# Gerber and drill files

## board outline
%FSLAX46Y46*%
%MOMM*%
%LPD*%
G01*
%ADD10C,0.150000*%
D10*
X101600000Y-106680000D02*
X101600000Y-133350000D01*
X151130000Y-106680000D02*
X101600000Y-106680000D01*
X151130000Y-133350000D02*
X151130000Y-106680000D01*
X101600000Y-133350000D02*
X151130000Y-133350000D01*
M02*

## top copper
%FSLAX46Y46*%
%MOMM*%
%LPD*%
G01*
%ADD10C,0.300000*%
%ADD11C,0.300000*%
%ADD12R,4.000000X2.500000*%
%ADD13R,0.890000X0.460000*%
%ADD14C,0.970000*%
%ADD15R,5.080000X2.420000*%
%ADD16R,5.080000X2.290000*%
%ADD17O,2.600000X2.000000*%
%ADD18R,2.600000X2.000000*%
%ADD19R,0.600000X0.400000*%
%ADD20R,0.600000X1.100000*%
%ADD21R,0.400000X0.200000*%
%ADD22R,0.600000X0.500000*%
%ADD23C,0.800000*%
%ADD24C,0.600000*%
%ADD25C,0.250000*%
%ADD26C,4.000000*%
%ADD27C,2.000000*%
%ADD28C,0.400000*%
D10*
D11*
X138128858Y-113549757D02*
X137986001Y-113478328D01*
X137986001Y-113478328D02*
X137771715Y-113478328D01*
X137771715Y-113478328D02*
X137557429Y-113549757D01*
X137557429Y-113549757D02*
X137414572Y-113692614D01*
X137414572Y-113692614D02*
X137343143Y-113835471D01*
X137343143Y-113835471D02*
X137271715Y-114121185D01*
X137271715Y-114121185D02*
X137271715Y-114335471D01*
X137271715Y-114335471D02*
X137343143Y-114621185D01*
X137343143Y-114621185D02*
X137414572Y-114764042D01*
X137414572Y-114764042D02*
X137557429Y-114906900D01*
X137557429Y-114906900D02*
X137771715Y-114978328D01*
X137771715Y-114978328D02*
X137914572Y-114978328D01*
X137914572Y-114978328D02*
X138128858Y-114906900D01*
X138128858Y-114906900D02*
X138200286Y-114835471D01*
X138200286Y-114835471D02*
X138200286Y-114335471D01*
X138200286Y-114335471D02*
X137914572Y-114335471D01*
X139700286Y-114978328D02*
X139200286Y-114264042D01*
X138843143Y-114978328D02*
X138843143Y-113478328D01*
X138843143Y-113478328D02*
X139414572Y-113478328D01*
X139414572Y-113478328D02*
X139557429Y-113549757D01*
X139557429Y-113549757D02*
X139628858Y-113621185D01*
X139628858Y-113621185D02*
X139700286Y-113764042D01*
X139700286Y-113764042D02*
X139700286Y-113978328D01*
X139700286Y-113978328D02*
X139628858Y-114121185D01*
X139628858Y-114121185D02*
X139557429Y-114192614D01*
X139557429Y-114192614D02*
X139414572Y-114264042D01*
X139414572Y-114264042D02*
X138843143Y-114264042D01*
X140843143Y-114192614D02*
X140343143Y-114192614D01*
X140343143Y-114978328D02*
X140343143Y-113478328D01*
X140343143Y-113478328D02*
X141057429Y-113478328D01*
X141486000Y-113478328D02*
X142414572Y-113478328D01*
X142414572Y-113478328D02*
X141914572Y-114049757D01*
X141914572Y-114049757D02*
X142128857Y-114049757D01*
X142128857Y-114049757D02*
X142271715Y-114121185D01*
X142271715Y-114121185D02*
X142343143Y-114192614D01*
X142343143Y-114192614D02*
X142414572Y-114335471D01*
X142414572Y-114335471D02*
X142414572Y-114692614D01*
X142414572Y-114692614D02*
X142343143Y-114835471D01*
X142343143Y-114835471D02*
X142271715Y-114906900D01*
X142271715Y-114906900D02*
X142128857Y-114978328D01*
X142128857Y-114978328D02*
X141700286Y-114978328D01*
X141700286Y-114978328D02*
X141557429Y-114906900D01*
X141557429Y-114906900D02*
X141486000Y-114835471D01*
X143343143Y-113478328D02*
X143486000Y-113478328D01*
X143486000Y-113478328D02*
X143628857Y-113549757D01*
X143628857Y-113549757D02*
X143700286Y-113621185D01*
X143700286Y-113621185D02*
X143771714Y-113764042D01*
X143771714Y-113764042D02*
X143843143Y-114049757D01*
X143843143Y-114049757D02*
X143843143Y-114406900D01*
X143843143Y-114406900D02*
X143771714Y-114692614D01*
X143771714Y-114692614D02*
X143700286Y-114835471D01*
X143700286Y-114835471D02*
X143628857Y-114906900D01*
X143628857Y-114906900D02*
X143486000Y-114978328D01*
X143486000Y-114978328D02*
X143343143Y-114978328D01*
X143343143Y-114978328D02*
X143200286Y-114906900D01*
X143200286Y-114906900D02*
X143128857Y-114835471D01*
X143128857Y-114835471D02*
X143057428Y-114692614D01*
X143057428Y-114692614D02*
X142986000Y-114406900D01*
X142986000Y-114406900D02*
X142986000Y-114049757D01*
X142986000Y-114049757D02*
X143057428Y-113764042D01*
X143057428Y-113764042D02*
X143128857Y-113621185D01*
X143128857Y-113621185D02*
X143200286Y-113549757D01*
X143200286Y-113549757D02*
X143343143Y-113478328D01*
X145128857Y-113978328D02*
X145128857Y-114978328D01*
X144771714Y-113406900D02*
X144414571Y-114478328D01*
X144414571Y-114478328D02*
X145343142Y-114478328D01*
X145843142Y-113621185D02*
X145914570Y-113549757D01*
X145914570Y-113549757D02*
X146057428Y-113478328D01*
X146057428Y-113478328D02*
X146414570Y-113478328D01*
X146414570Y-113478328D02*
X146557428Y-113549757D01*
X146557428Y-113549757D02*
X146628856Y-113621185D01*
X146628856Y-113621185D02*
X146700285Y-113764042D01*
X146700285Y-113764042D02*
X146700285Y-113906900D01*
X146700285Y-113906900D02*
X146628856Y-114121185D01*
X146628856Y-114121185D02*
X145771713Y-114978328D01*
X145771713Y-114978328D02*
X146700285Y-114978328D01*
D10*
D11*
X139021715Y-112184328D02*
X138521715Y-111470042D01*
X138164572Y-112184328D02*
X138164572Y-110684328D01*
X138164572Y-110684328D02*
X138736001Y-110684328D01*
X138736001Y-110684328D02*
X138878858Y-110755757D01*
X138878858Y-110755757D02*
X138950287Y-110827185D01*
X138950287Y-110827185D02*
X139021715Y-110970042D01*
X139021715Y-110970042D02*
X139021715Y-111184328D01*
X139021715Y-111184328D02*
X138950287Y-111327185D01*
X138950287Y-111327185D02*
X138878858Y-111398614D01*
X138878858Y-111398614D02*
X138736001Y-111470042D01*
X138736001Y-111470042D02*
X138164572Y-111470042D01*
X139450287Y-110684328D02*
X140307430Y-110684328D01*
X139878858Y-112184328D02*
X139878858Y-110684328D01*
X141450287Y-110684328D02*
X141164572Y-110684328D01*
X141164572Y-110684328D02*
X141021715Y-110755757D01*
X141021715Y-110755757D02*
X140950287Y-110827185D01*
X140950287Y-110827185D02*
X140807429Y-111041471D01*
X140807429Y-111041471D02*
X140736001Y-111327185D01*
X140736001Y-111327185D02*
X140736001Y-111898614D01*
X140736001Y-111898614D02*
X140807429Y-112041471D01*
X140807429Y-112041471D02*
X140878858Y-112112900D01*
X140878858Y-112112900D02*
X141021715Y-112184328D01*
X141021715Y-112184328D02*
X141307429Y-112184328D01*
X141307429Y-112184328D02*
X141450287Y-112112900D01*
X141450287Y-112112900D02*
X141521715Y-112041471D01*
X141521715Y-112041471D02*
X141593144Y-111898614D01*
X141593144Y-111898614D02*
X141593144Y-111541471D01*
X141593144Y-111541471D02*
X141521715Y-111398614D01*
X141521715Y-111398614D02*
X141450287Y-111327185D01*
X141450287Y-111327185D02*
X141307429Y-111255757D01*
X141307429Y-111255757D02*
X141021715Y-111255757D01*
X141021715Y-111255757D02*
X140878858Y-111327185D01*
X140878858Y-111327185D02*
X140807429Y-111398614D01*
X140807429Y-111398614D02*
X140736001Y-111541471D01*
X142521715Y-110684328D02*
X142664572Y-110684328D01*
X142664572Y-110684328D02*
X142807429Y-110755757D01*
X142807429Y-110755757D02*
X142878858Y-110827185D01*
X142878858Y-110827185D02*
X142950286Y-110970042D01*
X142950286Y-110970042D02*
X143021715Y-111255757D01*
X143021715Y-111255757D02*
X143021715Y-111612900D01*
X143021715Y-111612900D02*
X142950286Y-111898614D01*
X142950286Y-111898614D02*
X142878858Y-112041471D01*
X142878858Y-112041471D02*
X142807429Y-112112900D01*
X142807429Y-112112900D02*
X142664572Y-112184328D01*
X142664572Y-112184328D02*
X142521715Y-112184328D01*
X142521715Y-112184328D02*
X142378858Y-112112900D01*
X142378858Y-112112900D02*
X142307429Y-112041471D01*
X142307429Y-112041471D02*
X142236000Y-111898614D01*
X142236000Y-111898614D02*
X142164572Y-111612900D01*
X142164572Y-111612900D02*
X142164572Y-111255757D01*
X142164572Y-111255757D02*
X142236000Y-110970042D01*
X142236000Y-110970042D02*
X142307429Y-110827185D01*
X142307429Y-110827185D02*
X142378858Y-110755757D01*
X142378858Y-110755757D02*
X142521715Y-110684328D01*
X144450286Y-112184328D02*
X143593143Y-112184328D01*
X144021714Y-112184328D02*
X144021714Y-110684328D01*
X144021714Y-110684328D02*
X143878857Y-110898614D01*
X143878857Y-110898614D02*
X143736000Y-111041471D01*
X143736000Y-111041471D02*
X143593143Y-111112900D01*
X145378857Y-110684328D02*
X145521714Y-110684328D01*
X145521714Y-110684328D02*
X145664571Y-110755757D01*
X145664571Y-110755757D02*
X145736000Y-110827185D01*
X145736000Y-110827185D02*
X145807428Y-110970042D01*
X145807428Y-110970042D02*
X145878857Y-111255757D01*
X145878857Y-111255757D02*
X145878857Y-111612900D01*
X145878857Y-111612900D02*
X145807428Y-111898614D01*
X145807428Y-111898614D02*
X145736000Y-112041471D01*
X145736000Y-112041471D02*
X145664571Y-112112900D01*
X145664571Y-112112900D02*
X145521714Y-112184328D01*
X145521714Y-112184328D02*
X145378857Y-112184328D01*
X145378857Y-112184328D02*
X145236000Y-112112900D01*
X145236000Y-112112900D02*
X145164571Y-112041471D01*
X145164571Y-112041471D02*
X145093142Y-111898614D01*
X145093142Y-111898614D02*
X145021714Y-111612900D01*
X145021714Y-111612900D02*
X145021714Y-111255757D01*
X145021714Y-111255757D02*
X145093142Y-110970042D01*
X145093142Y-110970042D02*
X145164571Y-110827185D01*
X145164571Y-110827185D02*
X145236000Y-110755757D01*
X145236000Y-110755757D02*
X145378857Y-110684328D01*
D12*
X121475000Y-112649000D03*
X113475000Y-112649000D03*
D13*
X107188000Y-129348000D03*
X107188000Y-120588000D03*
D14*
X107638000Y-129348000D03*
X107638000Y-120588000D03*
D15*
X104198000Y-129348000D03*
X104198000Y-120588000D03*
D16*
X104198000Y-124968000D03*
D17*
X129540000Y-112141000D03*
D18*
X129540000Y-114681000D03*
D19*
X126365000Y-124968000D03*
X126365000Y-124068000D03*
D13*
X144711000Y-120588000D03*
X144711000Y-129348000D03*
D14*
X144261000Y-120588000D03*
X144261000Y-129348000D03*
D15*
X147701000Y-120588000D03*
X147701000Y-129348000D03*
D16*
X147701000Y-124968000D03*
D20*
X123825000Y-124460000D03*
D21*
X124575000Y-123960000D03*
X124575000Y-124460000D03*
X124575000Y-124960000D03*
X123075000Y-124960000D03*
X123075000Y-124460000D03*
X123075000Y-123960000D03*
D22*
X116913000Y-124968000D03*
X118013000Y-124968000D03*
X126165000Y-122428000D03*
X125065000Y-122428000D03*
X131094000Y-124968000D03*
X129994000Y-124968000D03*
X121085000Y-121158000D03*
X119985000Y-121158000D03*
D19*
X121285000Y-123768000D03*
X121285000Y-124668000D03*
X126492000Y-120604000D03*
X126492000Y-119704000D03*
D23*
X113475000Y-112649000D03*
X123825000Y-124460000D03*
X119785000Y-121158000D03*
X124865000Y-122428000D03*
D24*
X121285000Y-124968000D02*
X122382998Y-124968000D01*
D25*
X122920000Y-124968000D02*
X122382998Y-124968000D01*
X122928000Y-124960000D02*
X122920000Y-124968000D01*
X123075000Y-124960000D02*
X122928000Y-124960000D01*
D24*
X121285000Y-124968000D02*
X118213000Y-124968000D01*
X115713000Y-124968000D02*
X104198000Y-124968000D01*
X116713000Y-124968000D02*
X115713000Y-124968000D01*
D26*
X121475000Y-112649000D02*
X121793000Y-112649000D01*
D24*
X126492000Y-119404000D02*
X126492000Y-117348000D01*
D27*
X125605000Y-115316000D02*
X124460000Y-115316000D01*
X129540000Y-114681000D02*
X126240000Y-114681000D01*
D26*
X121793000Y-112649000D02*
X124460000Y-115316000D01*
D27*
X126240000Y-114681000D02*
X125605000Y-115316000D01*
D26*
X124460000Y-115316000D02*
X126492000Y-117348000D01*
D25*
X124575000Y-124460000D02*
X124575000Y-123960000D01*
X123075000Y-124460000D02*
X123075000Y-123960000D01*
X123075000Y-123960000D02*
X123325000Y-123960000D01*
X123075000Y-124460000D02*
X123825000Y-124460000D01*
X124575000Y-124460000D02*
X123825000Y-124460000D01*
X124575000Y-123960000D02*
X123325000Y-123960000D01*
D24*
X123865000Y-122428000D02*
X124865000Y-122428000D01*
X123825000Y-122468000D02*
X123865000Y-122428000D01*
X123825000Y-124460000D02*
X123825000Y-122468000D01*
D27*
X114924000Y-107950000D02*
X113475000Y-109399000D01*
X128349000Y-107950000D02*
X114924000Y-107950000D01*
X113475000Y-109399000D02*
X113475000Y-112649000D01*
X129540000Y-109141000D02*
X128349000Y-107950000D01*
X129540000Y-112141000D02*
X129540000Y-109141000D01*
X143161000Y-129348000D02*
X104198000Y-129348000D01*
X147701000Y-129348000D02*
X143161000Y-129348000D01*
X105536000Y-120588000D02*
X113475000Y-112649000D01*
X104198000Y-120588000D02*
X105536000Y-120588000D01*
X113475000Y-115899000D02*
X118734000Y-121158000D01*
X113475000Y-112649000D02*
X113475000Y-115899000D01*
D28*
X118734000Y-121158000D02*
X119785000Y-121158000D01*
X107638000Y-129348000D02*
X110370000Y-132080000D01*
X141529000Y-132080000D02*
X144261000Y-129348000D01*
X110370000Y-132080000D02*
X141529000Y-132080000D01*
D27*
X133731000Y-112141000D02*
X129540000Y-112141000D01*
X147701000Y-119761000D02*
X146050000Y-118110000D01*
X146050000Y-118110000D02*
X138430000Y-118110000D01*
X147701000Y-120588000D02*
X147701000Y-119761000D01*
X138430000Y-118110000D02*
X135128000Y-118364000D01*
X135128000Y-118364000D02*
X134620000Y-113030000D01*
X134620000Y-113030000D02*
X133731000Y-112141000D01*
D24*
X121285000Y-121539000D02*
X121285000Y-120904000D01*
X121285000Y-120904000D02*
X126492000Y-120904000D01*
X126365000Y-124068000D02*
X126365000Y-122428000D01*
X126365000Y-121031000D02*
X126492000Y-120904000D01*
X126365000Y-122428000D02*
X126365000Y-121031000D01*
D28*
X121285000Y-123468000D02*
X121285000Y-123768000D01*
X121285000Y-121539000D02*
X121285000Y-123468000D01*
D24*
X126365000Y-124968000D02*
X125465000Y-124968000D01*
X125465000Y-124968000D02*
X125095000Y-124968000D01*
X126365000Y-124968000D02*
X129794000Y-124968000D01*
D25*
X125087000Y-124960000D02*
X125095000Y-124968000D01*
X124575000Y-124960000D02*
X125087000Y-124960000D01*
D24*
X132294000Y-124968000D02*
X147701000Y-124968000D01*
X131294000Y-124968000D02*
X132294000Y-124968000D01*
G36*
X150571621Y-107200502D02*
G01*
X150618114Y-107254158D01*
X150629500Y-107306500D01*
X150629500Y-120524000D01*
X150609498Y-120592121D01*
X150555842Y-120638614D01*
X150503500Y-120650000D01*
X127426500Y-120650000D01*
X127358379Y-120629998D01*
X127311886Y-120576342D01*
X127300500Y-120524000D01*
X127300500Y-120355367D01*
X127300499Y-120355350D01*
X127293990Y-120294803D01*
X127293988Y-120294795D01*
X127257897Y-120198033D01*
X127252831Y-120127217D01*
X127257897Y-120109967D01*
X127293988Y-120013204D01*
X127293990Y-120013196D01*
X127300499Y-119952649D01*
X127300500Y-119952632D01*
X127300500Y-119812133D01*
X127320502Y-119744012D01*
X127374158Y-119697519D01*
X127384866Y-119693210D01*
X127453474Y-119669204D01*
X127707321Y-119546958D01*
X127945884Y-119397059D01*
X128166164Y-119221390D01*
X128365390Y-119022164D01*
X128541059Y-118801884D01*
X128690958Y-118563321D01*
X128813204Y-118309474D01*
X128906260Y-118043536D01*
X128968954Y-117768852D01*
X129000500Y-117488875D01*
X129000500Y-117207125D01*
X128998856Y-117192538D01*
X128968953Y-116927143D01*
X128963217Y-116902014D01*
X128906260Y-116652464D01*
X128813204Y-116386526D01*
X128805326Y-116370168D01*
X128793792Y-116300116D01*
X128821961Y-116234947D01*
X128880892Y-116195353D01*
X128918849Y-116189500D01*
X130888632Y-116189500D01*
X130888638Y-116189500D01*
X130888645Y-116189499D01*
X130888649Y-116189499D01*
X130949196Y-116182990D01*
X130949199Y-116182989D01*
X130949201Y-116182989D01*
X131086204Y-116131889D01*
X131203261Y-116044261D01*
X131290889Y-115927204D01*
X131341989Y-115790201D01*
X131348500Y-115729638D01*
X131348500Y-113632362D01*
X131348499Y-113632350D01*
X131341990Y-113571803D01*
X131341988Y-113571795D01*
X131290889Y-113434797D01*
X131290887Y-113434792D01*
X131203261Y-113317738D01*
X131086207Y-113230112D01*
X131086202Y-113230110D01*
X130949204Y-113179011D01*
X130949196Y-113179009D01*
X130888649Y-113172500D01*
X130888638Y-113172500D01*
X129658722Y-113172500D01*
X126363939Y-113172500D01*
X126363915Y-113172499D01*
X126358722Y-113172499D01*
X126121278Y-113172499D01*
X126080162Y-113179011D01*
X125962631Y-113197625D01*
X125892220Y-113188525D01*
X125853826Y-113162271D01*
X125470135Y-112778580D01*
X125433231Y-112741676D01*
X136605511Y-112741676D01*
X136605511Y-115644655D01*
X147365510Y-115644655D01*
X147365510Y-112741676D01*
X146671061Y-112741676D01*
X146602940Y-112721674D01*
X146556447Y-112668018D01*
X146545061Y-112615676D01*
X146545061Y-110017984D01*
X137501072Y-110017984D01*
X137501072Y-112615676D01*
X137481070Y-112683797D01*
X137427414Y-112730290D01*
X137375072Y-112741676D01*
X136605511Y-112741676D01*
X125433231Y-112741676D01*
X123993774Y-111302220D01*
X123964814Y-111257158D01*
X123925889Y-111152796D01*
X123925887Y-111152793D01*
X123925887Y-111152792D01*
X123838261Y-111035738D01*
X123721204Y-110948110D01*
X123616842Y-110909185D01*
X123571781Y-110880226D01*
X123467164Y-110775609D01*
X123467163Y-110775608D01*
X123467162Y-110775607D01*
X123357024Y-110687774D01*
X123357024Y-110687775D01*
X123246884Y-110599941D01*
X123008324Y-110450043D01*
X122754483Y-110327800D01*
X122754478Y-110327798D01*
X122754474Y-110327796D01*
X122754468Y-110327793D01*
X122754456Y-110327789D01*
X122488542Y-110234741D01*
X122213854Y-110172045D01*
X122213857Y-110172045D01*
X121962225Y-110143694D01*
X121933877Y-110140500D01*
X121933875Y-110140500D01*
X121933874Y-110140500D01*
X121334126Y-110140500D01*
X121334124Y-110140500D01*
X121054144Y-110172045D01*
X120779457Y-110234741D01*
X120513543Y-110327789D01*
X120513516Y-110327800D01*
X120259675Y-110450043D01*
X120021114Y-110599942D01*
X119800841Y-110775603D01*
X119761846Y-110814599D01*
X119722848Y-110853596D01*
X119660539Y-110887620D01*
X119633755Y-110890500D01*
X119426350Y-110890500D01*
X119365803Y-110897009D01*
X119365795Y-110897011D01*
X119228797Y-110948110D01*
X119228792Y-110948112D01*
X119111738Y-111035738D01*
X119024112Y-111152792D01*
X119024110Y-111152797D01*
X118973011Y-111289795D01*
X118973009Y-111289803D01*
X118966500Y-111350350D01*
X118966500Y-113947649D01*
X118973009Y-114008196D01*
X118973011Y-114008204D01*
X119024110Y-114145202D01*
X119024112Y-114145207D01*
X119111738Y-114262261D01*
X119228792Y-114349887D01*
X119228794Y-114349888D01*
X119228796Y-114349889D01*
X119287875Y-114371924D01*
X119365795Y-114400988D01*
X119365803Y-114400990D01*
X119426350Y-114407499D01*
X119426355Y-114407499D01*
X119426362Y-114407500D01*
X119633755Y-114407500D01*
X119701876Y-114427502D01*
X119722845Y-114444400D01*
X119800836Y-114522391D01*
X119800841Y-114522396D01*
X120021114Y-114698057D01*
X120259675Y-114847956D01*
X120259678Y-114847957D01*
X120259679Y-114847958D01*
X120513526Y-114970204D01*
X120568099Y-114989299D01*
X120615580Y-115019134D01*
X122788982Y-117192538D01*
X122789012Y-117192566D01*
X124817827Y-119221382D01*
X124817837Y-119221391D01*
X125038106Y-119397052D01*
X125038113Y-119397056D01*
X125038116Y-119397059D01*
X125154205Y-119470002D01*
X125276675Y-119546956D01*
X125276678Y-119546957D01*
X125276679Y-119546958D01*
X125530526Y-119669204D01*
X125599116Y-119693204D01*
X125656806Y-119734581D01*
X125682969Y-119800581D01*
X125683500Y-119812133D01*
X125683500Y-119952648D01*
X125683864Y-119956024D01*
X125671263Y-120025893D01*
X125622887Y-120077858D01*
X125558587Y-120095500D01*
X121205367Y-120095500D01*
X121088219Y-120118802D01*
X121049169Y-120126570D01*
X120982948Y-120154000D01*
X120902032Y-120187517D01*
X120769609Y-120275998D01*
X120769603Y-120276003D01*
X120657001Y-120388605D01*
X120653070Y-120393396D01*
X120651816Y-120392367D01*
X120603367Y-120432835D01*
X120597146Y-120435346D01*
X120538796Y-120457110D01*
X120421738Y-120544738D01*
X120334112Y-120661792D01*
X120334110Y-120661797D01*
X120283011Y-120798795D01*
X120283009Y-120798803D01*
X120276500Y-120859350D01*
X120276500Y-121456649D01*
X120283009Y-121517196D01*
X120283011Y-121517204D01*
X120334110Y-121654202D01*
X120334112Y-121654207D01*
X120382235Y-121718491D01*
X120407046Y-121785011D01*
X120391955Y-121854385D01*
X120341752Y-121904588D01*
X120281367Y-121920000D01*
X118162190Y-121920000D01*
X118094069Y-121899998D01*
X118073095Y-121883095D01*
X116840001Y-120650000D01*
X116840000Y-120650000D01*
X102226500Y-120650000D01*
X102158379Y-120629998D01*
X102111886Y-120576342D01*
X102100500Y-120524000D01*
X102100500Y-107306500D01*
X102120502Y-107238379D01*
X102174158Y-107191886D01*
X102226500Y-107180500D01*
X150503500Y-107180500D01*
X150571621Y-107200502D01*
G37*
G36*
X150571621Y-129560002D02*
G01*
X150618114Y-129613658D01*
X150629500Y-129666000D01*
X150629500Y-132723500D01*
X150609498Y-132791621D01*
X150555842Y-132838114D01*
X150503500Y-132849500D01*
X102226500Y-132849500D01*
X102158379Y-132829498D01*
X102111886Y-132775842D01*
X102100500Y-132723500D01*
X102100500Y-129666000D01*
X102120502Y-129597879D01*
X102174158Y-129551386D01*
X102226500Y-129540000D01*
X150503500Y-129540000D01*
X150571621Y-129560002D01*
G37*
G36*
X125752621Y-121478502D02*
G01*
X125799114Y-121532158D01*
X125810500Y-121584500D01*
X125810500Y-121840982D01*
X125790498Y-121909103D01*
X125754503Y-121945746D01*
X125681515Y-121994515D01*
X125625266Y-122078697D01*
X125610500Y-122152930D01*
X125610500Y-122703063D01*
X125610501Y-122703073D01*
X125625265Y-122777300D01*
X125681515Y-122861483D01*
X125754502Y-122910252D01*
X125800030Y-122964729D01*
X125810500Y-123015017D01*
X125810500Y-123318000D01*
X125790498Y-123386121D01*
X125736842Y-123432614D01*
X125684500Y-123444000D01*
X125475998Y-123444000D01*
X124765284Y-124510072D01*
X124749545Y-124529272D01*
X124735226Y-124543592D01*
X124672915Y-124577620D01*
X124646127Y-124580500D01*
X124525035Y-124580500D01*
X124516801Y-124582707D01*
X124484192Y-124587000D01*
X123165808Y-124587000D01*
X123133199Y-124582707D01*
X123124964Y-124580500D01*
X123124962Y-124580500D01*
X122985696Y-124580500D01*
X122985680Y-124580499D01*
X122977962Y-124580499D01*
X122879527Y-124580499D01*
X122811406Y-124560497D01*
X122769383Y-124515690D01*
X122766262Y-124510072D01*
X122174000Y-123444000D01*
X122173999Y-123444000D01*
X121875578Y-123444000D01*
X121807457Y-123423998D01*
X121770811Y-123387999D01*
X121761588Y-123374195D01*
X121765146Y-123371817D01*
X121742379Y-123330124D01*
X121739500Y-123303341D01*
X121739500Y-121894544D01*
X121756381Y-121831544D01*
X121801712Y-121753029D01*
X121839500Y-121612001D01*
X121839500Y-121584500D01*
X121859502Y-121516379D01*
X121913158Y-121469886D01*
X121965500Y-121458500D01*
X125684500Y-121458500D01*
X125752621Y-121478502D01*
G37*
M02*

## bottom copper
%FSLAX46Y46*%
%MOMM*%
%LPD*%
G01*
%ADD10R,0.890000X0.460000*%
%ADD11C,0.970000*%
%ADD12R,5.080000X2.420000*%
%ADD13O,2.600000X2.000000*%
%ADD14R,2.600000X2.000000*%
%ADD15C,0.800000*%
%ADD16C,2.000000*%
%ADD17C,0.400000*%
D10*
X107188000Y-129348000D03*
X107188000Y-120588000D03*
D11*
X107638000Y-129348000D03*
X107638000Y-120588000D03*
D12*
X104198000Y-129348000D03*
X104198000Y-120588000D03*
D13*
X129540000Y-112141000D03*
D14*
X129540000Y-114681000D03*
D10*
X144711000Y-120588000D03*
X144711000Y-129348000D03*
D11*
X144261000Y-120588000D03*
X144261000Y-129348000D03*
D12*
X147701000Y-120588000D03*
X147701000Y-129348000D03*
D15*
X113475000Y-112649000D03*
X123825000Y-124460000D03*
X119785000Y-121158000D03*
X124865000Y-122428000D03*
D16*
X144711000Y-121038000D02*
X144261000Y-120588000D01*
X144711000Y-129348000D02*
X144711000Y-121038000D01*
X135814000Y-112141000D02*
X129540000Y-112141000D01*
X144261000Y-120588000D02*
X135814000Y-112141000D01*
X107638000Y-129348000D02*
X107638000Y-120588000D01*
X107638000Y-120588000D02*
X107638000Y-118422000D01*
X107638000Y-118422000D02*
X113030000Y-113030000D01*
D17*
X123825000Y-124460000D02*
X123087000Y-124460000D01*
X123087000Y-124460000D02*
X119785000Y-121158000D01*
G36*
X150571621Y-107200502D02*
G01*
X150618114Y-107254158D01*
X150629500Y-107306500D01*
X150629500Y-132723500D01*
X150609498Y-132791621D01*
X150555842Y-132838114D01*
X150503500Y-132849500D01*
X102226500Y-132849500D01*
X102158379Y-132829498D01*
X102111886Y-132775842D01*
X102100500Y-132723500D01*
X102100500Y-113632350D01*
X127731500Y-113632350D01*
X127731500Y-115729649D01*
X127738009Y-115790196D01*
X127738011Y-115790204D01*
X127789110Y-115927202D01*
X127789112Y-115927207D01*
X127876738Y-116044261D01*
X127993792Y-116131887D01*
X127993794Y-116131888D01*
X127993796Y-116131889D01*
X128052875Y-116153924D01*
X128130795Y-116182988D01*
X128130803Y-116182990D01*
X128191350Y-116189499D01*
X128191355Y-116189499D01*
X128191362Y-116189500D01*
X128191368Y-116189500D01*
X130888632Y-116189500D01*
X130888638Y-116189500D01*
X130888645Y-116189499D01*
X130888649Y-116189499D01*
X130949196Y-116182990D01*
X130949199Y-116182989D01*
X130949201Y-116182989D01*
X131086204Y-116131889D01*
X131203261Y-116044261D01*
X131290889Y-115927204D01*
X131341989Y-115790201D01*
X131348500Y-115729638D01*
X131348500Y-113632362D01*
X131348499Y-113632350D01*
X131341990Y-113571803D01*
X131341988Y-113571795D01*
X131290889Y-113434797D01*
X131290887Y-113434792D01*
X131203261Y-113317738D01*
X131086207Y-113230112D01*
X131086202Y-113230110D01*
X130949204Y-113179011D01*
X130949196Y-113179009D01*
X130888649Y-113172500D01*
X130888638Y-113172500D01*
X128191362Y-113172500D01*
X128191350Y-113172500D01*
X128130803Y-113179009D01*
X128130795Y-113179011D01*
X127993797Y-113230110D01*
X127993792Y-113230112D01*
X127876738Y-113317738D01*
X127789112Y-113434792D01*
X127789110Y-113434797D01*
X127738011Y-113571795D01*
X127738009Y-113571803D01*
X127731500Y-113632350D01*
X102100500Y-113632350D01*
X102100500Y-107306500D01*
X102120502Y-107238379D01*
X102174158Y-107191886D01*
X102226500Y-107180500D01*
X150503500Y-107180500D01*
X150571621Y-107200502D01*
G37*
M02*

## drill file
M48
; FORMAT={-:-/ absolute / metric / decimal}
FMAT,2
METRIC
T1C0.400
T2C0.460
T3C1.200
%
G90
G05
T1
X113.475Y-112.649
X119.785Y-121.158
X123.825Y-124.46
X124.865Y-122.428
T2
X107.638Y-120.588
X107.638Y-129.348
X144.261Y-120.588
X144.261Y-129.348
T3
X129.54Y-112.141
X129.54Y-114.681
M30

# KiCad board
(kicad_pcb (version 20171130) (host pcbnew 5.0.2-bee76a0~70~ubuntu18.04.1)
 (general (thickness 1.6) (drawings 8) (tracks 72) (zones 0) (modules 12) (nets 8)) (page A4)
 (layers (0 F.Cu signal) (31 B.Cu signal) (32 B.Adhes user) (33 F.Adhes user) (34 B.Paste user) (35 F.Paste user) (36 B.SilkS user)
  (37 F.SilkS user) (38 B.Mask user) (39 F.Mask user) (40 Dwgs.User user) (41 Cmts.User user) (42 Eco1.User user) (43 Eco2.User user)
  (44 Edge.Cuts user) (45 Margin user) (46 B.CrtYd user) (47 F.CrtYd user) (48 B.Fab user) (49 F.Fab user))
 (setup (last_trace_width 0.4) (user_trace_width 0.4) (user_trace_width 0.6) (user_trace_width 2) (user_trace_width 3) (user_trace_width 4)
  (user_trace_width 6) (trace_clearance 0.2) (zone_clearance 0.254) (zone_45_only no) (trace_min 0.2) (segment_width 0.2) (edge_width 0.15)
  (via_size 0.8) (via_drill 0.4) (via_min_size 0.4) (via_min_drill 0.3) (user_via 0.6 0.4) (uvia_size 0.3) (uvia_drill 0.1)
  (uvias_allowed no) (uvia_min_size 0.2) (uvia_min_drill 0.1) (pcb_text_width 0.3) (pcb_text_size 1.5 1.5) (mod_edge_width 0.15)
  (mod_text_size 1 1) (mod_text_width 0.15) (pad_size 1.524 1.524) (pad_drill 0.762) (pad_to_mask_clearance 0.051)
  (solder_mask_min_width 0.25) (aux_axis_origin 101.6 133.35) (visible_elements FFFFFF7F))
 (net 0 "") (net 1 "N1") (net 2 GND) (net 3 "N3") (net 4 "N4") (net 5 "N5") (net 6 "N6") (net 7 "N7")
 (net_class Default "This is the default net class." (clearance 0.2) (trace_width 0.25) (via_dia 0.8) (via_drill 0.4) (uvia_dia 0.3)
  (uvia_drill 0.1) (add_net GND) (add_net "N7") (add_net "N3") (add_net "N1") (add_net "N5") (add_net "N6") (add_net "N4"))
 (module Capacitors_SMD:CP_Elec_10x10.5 (layer F.Cu) (at 117.475 112.649)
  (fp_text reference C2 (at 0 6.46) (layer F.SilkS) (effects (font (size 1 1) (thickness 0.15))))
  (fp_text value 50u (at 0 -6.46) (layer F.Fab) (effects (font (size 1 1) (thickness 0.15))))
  (pad 2 smd rect (at 4 0 180) (size 4 2.5) (layers F.Cu F.Paste F.Mask) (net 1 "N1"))
  (pad 1 smd rect (at -4 0 180) (size 4 2.5) (layers F.Cu F.Paste F.Mask) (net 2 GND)))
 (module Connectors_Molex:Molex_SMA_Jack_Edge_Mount (layer F.Cu) (at 105.918 124.968)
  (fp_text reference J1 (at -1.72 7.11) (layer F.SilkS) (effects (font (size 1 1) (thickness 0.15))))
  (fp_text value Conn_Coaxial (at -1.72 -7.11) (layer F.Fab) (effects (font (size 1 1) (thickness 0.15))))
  (pad 2 smd rect (at 1.27 4.38) (size 0.89 0.46) (layers B.Cu) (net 2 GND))
  (pad 2 smd rect (at 1.27 -4.38) (size 0.89 0.46) (layers B.Cu) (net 2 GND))
  (pad 2 smd rect (at 1.27 4.38) (size 0.89 0.46) (layers F.Cu) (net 2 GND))
  (pad 2 smd rect (at 1.27 -4.38) (size 0.89 0.46) (layers F.Cu) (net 2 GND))
  (pad 2 thru_hole circle (at 1.72 4.38) (size 0.97 0.97) (drill 0.46) (layers *.Cu) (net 2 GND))
  (pad 2 thru_hole circle (at 1.72 -4.38) (size 0.97 0.97) (drill 0.46) (layers *.Cu) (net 2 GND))
  (pad 2 smd rect (at -1.72 4.38) (size 5.08 2.42) (layers B.Cu B.Paste B.Mask) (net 2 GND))
  (pad 2 smd rect (at -1.72 -4.38) (size 5.08 2.42) (layers B.Cu B.Paste B.Mask) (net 2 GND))
  (pad 2 smd rect (at -1.72 4.38) (size 5.08 2.42) (layers F.Cu F.Paste F.Mask) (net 2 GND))
  (pad 2 smd rect (at -1.72 -4.38) (size 5.08 2.42) (layers F.Cu F.Paste F.Mask) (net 2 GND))
  (pad 1 smd rect (at -1.72 0) (size 5.08 2.29) (layers F.Cu F.Paste F.Mask) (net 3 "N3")))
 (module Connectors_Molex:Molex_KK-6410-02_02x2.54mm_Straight (layer F.Cu) (at 129.54 114.681 90)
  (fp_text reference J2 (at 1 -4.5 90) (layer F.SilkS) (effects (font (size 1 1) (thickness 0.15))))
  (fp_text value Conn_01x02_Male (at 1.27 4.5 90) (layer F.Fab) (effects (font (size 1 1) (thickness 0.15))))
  (pad 2 thru_hole oval (at 2.54 0 90) (size 2 2.6) (drill 1.2) (layers *.Cu *.Mask) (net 2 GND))
  (pad 1 thru_hole rect (at 0 0 90) (size 2 2.6) (drill 1.2) (layers *.Cu *.Mask) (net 1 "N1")))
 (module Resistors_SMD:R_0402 (layer F.Cu) (at 126.365 124.518 270)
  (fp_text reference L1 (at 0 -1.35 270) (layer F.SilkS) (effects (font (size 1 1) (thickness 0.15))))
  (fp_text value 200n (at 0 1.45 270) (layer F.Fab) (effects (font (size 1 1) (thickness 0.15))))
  (pad 2 smd rect (at 0.45 0 270) (size 0.4 0.6) (layers F.Cu F.Paste F.Mask) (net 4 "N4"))
  (pad 1 smd rect (at -0.45 0 270) (size 0.4 0.6) (layers F.Cu F.Paste F.Mask) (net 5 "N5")))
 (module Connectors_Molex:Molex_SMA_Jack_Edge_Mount (layer F.Cu) (at 145.981 124.968 180)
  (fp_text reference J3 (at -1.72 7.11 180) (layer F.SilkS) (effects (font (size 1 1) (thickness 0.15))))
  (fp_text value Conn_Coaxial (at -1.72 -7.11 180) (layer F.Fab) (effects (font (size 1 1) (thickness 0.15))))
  (pad 2 smd rect (at 1.27 4.38 180) (size 0.89 0.46) (layers B.Cu) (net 2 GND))
  (pad 2 smd rect (at 1.27 -4.38 180) (size 0.89 0.46) (layers B.Cu) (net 2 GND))
  (pad 2 smd rect (at 1.27 4.38 180) (size 0.89 0.46) (layers F.Cu) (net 2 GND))
  (pad 2 smd rect (at 1.27 -4.38 180) (size 0.89 0.46) (layers F.Cu) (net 2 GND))
  (pad 2 thru_hole circle (at 1.72 4.38 180) (size 0.97 0.97) (drill 0.46) (layers *.Cu) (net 2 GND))
  (pad 2 thru_hole circle (at 1.72 -4.38 180) (size 0.97 0.97) (drill 0.46) (layers *.Cu) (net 2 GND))
  (pad 2 smd rect (at -1.72 4.38 180) (size 5.08 2.42) (layers B.Cu B.Paste B.Mask) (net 2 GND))
  (pad 2 smd rect (at -1.72 -4.38 180) (size 5.08 2.42) (layers B.Cu B.Paste B.Mask) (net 2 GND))
  (pad 2 smd rect (at -1.72 4.38 180) (size 5.08 2.42) (layers F.Cu F.Paste F.Mask) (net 2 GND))
  (pad 2 smd rect (at -1.72 -4.38 180) (size 5.08 2.42) (layers F.Cu F.Paste F.Mask) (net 2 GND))
  (pad 1 smd rect (at -1.72 0 180) (size 5.08 2.29) (layers F.Cu F.Paste F.Mask) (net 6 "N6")))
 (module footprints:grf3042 (layer F.Cu) (at 123.825 124.46)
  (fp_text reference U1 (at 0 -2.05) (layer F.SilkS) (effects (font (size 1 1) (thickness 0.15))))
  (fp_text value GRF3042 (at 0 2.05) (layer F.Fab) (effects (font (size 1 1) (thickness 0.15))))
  (pad 7 smd rect (at 0 0) (size 0.6 1.1) (layers F.Cu F.Paste F.Mask) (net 2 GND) (solder_paste_margin_ratio -0.2))
  (pad 6 smd rect (at 0.75 -0.5) (size 0.4 0.2) (layers F.Cu F.Paste F.Mask) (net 2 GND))
  (pad 5 smd rect (at 0.75 0) (size 0.4 0.2) (layers F.Cu F.Paste F.Mask) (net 2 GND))
  (pad 4 smd rect (at 0.75 0.5) (size 0.4 0.2) (layers F.Cu F.Paste F.Mask) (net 4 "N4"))
  (pad 3 smd rect (at -0.75 0.5) (size 0.4 0.2) (layers F.Cu F.Paste F.Mask) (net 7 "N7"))
  (pad 2 smd rect (at -0.75 0) (size 0.4 0.2) (layers F.Cu F.Paste F.Mask) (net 2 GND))
  (pad 1 smd rect (at -0.75 -0.5) (size 0.4 0.2) (layers F.Cu F.Paste F.Mask) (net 2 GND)))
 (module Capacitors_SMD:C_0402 (layer F.Cu) (at 117.463 124.968 180)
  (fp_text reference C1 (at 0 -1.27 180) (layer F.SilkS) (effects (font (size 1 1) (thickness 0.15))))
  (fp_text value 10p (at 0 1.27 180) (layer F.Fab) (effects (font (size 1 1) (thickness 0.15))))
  (pad 2 smd rect (at 0.55 0 180) (size 0.6 0.5) (layers F.Cu F.Paste F.Mask) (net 3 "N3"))
  (pad 1 smd rect (at -0.55 0 180) (size 0.6 0.5) (layers F.Cu F.Paste F.Mask) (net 7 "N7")))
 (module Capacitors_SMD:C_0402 (layer F.Cu) (at 125.615 122.428)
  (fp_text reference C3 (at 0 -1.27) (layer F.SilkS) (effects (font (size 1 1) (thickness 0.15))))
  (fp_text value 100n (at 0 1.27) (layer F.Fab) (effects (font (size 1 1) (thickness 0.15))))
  (pad 2 smd rect (at 0.55 0) (size 0.6 0.5) (layers F.Cu F.Paste F.Mask) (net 5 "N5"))
  (pad 1 smd rect (at -0.55 0) (size 0.6 0.5) (layers F.Cu F.Paste F.Mask) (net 2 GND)))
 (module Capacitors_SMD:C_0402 (layer F.Cu) (at 130.544 124.968 180)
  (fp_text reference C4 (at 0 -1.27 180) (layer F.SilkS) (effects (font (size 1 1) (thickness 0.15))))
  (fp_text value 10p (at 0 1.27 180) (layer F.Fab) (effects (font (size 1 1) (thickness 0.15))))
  (pad 1 smd rect (at -0.55 0 180) (size 0.6 0.5) (layers F.Cu F.Paste F.Mask) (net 6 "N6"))
  (pad 2 smd rect (at 0.55 0 180) (size 0.6 0.5) (layers F.Cu F.Paste F.Mask) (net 4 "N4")))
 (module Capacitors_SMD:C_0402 (layer F.Cu) (at 120.535 121.158 180)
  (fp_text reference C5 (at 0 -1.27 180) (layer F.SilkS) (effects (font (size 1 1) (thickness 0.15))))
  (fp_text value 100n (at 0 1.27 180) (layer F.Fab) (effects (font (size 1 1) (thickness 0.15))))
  (pad 1 smd rect (at -0.55 0 180) (size 0.6 0.5) (layers F.Cu F.Paste F.Mask) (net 5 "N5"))
  (pad 2 smd rect (at 0.55 0 180) (size 0.6 0.5) (layers F.Cu F.Paste F.Mask) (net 2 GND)))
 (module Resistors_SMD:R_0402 (layer F.Cu) (at 121.285 124.218 270)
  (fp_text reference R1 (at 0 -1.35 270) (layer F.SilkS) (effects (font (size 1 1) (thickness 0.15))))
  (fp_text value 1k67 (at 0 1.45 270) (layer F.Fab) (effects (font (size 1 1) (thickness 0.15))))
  (pad 1 smd rect (at -0.45 0 270) (size 0.4 0.6) (layers F.Cu F.Paste F.Mask) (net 5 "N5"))
  (pad 2 smd rect (at 0.45 0 270) (size 0.4 0.6) (layers F.Cu F.Paste F.Mask) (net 7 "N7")))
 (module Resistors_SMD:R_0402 (layer F.Cu) (at 126.492 120.154 270)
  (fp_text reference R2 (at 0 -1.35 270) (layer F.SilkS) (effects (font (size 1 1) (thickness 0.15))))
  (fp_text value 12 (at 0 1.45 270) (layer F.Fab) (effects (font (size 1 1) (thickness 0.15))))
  (pad 2 smd rect (at 0.45 0 270) (size 0.4 0.6) (layers F.Cu F.Paste F.Mask) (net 5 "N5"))
  (pad 1 smd rect (at -0.45 0 270) (size 0.4 0.6) (layers F.Cu F.Paste F.Mask) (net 1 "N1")))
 (gr_line (start 101.6 106.68) (end 101.6 133.35) (layer Edge.Cuts) (width 0.15))
 (gr_line (start 151.13 106.68) (end 101.6 106.68) (layer Edge.Cuts) (width 0.15))
 (gr_line (start 151.13 133.35) (end 151.13 106.68) (layer Edge.Cuts) (width 0.15))
 (gr_line (start 101.6 133.35) (end 151.13 133.35) (layer Edge.Cuts) (width 0.15))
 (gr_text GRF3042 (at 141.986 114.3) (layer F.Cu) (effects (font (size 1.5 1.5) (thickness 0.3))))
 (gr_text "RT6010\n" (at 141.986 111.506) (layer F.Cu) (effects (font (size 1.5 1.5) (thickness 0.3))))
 (segment (start 121.285 124.968) (end 122.382998 124.968) (width 0.6) (layer F.Cu) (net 7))
 (segment (start 122.92 124.968) (end 122.382998 124.968) (width 0.25) (layer F.Cu) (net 7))
 (segment (start 122.928 124.96) (end 122.92 124.968) (width 0.25) (layer F.Cu) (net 7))
 (segment (start 123.075 124.96) (end 122.928 124.96) (width 0.25) (layer F.Cu) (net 7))
 (segment (start 121.285 124.968) (end 118.213 124.968) (width 0.6) (layer F.Cu) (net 7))
 (segment (start 115.713 124.968) (end 104.198 124.968) (width 0.6) (layer F.Cu) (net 3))
 (segment (start 116.713 124.968) (end 115.713 124.968) (width 0.6) (layer F.Cu) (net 3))
 (segment (start 121.475 112.649) (end 121.793 112.649) (width 4) (layer F.Cu) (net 1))
 (segment (start 126.492 119.404) (end 126.492 117.348) (width 0.6) (layer F.Cu) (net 1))
 (segment (start 125.605 115.316) (end 124.46 115.316) (width 2) (layer F.Cu) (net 1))
 (segment (start 129.54 114.681) (end 126.24 114.681) (width 2) (layer F.Cu) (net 1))
 (segment (start 121.793 112.649) (end 124.46 115.316) (width 4) (layer F.Cu) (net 1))
 (segment (start 126.24 114.681) (end 125.605 115.316) (width 2) (layer F.Cu) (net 1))
 (segment (start 124.46 115.316) (end 126.492 117.348) (width 4) (layer F.Cu) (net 1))
 (segment (start 124.575 124.46) (end 124.575 123.96) (width 0.25) (layer F.Cu) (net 2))
 (segment (start 123.075 124.46) (end 123.075 123.96) (width 0.25) (layer F.Cu) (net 2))
 (segment (start 123.075 123.96) (end 123.325 123.96) (width 0.25) (layer F.Cu) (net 2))
 (segment (start 123.075 124.46) (end 123.825 124.46) (width 0.25) (layer F.Cu) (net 2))
 (segment (start 124.575 124.46) (end 123.825 124.46) (width 0.25) (layer F.Cu) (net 2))
 (segment (start 124.575 123.96) (end 123.325 123.96) (width 0.25) (layer F.Cu) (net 2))
 (segment (start 123.865 122.428) (end 124.865 122.428) (width 0.6) (layer F.Cu) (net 2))
 (segment (start 123.825 122.468) (end 123.865 122.428) (width 0.6) (layer F.Cu) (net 2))
 (segment (start 123.825 124.46) (end 123.825 122.468) (width 0.6) (layer F.Cu) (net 2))
 (segment (start 144.711 121.038) (end 144.261 120.588) (width 2) (layer B.Cu) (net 2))
 (segment (start 144.711 129.348) (end 144.711 121.038) (width 2) (layer B.Cu) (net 2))
 (segment (start 135.814 112.141) (end 129.54 112.141) (width 2) (layer B.Cu) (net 2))
 (segment (start 144.261 120.588) (end 135.814 112.141) (width 2) (layer B.Cu) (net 2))
 (segment (start 107.638 129.348) (end 107.638 120.588) (width 2) (layer B.Cu) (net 2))
 (segment (start 107.638 120.588) (end 107.638 118.422) (width 2) (layer B.Cu) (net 2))
 (segment (start 107.638 118.422) (end 113.03 113.03) (width 2) (layer B.Cu) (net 2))
 (segment (start 114.924 107.95) (end 113.475 109.399) (width 2) (layer F.Cu) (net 2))
 (segment (start 128.349 107.95) (end 114.924 107.95) (width 2) (layer F.Cu) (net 2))
 (segment (start 113.475 109.399) (end 113.475 112.649) (width 2) (layer F.Cu) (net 2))
 (segment (start 129.54 109.141) (end 128.349 107.95) (width 2) (layer F.Cu) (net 2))
 (segment (start 129.54 112.141) (end 129.54 109.141) (width 2) (layer F.Cu) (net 2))
 (segment (start 143.161 129.348) (end 104.198 129.348) (width 2) (layer F.Cu) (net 2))
 (segment (start 147.701 129.348) (end 143.161 129.348) (width 2) (layer F.Cu) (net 2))
 (segment (start 105.536 120.588) (end 113.475 112.649) (width 2) (layer F.Cu) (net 2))
 (segment (start 104.198 120.588) (end 105.536 120.588) (width 2) (layer F.Cu) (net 2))
 (segment (start 113.475 115.899) (end 118.734 121.158) (width 2) (layer F.Cu) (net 2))
 (segment (start 113.475 112.649) (end 113.475 115.899) (width 2) (layer F.Cu) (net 2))
 (segment (start 118.734 121.158) (end 119.785 121.158) (width 0.4) (layer F.Cu) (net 2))
 (via (at 113.475 112.649) (size 0.8) (drill 0.4) (layers F.Cu B.Cu) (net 2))
 (via (at 123.825 124.46) (size 0.8) (drill 0.4) (layers F.Cu B.Cu) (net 2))
 (via (at 119.785 121.158) (size 0.8) (drill 0.4) (layers F.Cu B.Cu) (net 2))
 (segment (start 123.825 124.46) (end 123.087 124.46) (width 0.4) (layer B.Cu) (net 2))
 (segment (start 123.087 124.46) (end 119.785 121.158) (width 0.4) (layer B.Cu) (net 2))
 (via (at 124.865 122.428) (size 0.8) (drill 0.4) (layers F.Cu B.Cu) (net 2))
 (segment (start 107.638 129.348) (end 110.37 132.08) (width 0.4) (layer F.Cu) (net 2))
 (segment (start 141.529 132.08) (end 144.261 129.348) (width 0.4) (layer F.Cu) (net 2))
 (segment (start 110.37 132.08) (end 141.529 132.08) (width 0.4) (layer F.Cu) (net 2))
 (segment (start 133.731 112.141) (end 129.54 112.141) (width 2) (layer F.Cu) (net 2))
 (segment (start 147.701 119.761) (end 146.05 118.11) (width 2) (layer F.Cu) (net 2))
 (segment (start 146.05 118.11) (end 138.43 118.11) (width 2) (layer F.Cu) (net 2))
 (segment (start 147.701 120.588) (end 147.701 119.761) (width 2) (layer F.Cu) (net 2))
 (segment (start 138.43 118.11) (end 135.128 118.364) (width 2) (layer F.Cu) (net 2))
 (segment (start 135.128 118.364) (end 134.62 113.03) (width 2) (layer F.Cu) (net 2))
 (segment (start 134.62 113.03) (end 133.731 112.141) (width 2) (layer F.Cu) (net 2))
 (segment (start 121.285 121.539) (end 121.285 120.904) (width 0.6) (layer F.Cu) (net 5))
 (segment (start 121.285 120.904) (end 126.492 120.904) (width 0.6) (layer F.Cu) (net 5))
 (segment (start 126.365 124.068) (end 126.365 122.428) (width 0.6) (layer F.Cu) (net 5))
 (segment (start 126.365 121.031) (end 126.492 120.904) (width 0.6) (layer F.Cu) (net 5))
 (segment (start 126.365 122.428) (end 126.365 121.031) (width 0.6) (layer F.Cu) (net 5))
 (segment (start 121.285 123.468) (end 121.285 123.768) (width 0.4) (layer F.Cu) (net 5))
 (segment (start 121.285 121.539) (end 121.285 123.468) (width 0.4) (layer F.Cu) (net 5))
 (segment (start 126.365 124.968) (end 125.465 124.968) (width 0.6) (layer F.Cu) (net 4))
 (segment (start 125.465 124.968) (end 125.095 124.968) (width 0.6) (layer F.Cu) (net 4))
 (segment (start 126.365 124.968) (end 129.794 124.968) (width 0.6) (layer F.Cu) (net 4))
 (segment (start 125.087 124.96) (end 125.095 124.968) (width 0.25) (layer F.Cu) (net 4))
 (segment (start 124.575 124.96) (end 125.087 124.96) (width 0.25) (layer F.Cu) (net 4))
 (segment (start 132.294 124.968) (end 147.701 124.968) (width 0.6) (layer F.Cu) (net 6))
 (segment (start 131.294 124.968) (end 132.294 124.968) (width 0.6) (layer F.Cu) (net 6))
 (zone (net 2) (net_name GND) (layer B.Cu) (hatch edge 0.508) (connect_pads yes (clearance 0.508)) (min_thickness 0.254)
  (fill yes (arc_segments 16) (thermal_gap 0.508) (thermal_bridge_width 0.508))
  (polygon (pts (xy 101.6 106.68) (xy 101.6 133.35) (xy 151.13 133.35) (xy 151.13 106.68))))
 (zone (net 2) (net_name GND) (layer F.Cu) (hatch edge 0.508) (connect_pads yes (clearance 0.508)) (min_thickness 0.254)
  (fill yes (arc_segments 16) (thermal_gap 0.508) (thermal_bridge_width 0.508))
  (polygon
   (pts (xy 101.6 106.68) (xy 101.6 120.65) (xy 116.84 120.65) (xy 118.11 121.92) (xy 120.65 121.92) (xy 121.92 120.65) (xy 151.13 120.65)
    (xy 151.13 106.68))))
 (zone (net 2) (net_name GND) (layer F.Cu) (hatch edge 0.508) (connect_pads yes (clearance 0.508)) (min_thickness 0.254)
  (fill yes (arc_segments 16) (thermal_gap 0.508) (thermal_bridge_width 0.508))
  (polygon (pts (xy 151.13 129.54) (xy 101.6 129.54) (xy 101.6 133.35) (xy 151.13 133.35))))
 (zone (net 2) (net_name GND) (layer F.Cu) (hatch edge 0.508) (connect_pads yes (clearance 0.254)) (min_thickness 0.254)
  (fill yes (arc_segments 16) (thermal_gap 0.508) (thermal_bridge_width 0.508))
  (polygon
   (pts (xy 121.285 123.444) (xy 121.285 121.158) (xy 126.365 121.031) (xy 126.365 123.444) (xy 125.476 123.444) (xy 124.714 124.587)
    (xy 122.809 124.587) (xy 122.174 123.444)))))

